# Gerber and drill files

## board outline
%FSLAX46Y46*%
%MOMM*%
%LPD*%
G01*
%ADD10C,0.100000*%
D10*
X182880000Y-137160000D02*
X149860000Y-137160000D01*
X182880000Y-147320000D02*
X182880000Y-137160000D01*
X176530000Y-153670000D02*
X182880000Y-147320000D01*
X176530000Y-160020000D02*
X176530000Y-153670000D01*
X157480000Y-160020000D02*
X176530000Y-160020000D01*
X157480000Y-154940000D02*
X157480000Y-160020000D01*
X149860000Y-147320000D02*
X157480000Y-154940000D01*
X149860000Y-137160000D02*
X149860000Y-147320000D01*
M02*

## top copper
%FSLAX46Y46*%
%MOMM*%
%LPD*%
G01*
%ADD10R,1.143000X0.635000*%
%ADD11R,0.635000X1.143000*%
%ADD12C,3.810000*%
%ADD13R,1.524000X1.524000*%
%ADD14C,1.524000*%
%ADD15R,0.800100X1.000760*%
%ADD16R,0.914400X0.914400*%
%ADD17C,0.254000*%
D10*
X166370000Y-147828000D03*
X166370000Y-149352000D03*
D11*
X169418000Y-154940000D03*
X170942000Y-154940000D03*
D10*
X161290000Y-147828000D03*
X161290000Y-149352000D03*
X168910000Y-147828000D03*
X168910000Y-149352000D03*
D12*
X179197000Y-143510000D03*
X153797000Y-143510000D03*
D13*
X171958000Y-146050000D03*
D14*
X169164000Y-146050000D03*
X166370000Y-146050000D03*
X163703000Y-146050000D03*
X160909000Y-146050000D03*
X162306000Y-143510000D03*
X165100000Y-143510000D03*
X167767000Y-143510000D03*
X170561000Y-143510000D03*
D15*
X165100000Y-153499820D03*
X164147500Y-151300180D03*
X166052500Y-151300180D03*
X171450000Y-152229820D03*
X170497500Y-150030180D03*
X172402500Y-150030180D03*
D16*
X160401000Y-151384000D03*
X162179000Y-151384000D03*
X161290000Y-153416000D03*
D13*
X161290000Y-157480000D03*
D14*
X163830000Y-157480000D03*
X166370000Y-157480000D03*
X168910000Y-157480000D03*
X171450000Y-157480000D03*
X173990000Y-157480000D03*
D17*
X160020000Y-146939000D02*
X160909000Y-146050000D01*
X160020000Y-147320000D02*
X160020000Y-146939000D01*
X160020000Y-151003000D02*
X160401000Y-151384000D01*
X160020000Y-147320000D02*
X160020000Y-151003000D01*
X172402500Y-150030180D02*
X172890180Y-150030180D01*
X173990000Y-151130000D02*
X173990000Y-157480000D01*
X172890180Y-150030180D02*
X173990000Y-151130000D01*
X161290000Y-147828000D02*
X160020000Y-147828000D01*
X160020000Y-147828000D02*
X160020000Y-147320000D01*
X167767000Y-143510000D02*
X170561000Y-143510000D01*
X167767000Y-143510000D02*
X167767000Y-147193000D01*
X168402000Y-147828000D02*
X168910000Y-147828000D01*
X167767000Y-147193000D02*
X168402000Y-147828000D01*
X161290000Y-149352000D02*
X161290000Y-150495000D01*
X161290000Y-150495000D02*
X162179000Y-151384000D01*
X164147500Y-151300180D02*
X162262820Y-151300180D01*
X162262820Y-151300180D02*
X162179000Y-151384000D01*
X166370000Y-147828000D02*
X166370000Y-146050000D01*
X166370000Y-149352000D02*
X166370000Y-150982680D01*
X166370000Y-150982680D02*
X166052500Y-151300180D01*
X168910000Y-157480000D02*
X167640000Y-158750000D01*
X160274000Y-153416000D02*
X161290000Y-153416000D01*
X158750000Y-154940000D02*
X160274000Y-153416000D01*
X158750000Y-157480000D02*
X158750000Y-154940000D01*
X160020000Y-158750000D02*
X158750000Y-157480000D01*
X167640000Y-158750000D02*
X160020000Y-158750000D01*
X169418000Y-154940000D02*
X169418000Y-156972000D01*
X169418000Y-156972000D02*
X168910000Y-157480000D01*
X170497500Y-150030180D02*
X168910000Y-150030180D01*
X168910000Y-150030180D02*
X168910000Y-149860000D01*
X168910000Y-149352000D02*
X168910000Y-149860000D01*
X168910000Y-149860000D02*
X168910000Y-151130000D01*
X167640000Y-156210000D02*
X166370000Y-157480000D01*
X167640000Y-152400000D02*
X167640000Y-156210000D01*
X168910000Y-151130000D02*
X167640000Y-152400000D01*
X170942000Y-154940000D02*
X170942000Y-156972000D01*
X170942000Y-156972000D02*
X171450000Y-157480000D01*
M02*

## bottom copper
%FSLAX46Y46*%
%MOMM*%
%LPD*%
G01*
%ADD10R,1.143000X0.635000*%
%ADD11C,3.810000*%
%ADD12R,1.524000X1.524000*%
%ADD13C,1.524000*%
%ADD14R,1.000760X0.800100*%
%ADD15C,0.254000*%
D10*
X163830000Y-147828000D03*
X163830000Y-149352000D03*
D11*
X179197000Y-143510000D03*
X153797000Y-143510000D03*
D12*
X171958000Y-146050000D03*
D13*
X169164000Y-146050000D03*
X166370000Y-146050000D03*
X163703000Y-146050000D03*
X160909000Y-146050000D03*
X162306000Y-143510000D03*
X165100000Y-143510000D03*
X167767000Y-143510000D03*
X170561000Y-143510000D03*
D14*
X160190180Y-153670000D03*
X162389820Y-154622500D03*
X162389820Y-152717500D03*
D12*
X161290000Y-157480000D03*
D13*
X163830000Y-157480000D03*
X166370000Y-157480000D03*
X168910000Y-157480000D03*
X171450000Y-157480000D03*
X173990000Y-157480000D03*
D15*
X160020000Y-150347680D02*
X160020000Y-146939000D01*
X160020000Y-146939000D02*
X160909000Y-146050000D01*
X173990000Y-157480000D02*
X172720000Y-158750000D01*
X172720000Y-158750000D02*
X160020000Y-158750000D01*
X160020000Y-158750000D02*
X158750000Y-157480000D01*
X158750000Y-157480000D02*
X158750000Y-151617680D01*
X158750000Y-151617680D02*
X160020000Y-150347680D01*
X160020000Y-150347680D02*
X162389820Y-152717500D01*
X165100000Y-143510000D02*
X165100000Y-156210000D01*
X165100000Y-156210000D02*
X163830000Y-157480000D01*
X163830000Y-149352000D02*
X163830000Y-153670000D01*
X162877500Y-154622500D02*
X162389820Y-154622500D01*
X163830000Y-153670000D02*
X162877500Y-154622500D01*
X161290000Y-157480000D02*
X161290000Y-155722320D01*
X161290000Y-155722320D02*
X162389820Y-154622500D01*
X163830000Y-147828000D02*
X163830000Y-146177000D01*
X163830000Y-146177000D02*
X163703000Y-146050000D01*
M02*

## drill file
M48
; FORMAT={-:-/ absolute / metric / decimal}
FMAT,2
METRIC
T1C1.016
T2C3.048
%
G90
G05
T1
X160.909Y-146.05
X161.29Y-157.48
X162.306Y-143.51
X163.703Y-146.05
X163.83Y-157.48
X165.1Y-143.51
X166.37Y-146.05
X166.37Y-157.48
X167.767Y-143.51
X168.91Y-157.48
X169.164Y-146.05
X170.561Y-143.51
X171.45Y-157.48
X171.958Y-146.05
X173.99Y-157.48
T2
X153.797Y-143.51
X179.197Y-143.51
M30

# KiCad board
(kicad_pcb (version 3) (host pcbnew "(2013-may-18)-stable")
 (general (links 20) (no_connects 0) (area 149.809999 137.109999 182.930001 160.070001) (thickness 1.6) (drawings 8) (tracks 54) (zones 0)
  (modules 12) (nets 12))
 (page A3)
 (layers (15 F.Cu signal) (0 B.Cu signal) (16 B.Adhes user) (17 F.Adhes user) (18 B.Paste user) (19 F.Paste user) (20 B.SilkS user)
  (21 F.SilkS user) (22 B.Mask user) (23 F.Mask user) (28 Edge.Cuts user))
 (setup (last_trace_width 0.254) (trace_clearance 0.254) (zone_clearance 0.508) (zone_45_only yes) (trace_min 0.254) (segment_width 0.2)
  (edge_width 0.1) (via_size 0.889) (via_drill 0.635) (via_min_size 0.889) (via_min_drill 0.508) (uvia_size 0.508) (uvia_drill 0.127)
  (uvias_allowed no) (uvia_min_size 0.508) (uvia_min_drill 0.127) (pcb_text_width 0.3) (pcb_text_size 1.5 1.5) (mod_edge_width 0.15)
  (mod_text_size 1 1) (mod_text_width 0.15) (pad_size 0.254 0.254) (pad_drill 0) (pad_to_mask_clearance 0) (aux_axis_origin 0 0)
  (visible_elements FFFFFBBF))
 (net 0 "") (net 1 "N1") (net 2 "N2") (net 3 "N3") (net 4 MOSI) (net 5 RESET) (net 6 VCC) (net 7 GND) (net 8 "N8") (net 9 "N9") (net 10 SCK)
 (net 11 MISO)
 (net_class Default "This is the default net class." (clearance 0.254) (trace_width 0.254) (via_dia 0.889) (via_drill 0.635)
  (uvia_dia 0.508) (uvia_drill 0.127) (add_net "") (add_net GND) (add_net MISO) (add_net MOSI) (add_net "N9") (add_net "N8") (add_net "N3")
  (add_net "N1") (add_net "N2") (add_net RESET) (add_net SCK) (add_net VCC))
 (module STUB (layer F.Cu) (at 0 0)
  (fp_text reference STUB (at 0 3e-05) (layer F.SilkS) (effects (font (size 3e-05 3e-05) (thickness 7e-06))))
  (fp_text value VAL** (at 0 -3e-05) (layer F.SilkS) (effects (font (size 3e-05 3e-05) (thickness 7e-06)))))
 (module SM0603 (layer F.Cu) (at 166.37 148.59 270)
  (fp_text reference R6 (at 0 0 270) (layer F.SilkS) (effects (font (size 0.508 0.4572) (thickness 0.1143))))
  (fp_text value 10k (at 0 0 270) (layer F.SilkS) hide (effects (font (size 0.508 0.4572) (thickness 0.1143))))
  (pad 1 smd rect (at -0.762 0 270) (size 0.635 1.143) (layers F.Cu F.Paste F.Mask) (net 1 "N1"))
  (pad 2 smd rect (at 0.762 0 270) (size 0.635 1.143) (layers F.Cu F.Paste F.Mask) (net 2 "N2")))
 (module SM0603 (layer B.Cu) (at 163.83 148.59 270)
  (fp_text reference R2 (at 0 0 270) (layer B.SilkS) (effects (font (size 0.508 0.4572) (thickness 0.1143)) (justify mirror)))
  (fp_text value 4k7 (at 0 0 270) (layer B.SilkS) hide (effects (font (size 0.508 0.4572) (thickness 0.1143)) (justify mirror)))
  (pad 1 smd rect (at -0.762 0 270) (size 0.635 1.143) (layers B.Cu B.Paste B.Mask) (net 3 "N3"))
  (pad 2 smd rect (at 0.762 0 270) (size 0.635 1.143) (layers B.Cu B.Paste B.Mask) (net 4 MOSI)))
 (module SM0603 (layer F.Cu) (at 170.18 154.94)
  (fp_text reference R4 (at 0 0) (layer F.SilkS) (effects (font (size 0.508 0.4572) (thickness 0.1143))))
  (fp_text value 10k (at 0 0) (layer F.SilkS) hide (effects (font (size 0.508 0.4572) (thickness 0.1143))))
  (pad 1 smd rect (at -0.762 0) (size 0.635 1.143) (layers F.Cu F.Paste F.Mask) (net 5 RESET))
  (pad 2 smd rect (at 0.762 0) (size 0.635 1.143) (layers F.Cu F.Paste F.Mask) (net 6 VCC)))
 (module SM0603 (layer F.Cu) (at 161.29 148.59 270)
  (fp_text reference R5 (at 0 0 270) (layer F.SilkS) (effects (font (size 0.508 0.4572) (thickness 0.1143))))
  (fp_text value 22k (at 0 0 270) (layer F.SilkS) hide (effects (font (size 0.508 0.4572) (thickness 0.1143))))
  (pad 1 smd rect (at -0.762 0 270) (size 0.635 1.143) (layers F.Cu F.Paste F.Mask) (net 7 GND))
  (pad 2 smd rect (at 0.762 0 270) (size 0.635 1.143) (layers F.Cu F.Paste F.Mask) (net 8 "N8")))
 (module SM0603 (layer F.Cu) (at 168.91 148.59 270)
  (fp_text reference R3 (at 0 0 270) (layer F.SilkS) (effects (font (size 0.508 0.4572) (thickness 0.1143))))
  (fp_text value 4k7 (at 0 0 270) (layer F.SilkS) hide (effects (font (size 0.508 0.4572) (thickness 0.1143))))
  (pad 1 smd rect (at -0.762 0 270) (size 0.635 1.143) (layers F.Cu F.Paste F.Mask) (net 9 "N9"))
  (pad 2 smd rect (at 0.762 0 270) (size 0.635 1.143) (layers F.Cu F.Paste F.Mask) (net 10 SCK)))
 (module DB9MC (layer F.Cu) (at 166.37 144.78)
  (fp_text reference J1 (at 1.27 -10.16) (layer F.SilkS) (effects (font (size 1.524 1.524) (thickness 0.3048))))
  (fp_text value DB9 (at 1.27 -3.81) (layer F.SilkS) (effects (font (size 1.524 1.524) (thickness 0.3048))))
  (pad "" thru_hole circle (at 12.827 -1.27) (size 3.81 3.81) (drill 3.048) (layers *.Cu *.Mask F.SilkS))
  (pad "" thru_hole circle (at -12.573 -1.27) (size 3.81 3.81) (drill 3.048) (layers *.Cu *.Mask F.SilkS))
  (pad 1 thru_hole rect (at 5.588 1.27) (size 1.524 1.524) (drill 1.016) (layers *.Cu *.Mask F.SilkS))
  (pad 2 thru_hole circle (at 2.794 1.27) (size 1.524 1.524) (drill 1.016) (layers *.Cu *.Mask F.SilkS))
  (pad 3 thru_hole circle (at 0 1.27) (size 1.524 1.524) (drill 1.016) (layers *.Cu *.Mask F.SilkS) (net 1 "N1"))
  (pad 4 thru_hole circle (at -2.667 1.27) (size 1.524 1.524) (drill 1.016) (layers *.Cu *.Mask F.SilkS) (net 3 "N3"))
  (pad 5 thru_hole circle (at -5.461 1.27) (size 1.524 1.524) (drill 1.016) (layers *.Cu *.Mask F.SilkS) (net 7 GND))
  (pad 9 thru_hole circle (at -4.064 -1.27) (size 1.524 1.524) (drill 1.016) (layers *.Cu *.Mask F.SilkS))
  (pad 8 thru_hole circle (at -1.27 -1.27) (size 1.524 1.524) (drill 1.016) (layers *.Cu *.Mask F.SilkS) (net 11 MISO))
  (pad 7 thru_hole circle (at 1.397 -1.27) (size 1.524 1.524) (drill 1.016) (layers *.Cu *.Mask F.SilkS) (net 9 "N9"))
  (pad 6 thru_hole circle (at 4.191 -1.27) (size 1.524 1.524) (drill 1.016) (layers *.Cu *.Mask F.SilkS) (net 9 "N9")))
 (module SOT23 (layer F.Cu) (at 165.1 152.4 180)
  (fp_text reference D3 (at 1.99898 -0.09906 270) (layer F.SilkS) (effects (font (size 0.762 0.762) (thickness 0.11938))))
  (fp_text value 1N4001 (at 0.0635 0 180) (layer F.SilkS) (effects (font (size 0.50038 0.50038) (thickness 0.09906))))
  (pad 3 smd rect (at 0 -1.09982 180) (size 0.8001 1.00076) (layers F.Cu F.Paste F.Mask))
  (pad 2 smd rect (at 0.9525 1.09982 180) (size 0.8001 1.00076) (layers F.Cu F.Paste F.Mask) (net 8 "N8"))
  (pad 1 smd rect (at -0.9525 1.09982 180) (size 0.8001 1.00076) (layers F.Cu F.Paste F.Mask) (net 2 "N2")))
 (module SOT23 (layer B.Cu) (at 161.29 153.67 270)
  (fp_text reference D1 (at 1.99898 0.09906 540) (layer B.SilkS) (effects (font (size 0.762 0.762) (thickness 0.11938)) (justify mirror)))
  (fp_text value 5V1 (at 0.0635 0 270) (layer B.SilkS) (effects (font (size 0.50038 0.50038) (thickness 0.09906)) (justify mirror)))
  (pad 3 smd rect (at 0 1.09982 270) (size 0.8001 1.00076) (layers B.Cu B.Paste B.Mask))
  (pad 2 smd rect (at 0.9525 -1.09982 270) (size 0.8001 1.00076) (layers B.Cu B.Paste B.Mask) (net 4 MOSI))
  (pad 1 smd rect (at -0.9525 -1.09982 270) (size 0.8001 1.00076) (layers B.Cu B.Paste B.Mask) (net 7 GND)))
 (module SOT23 (layer F.Cu) (at 171.45 151.13 180)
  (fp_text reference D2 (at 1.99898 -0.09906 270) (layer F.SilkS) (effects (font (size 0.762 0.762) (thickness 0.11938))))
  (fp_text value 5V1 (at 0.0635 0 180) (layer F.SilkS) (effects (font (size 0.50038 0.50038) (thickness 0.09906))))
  (pad 3 smd rect (at 0 -1.09982 180) (size 0.8001 1.00076) (layers F.Cu F.Paste F.Mask))
  (pad 2 smd rect (at 0.9525 1.09982 180) (size 0.8001 1.00076) (layers F.Cu F.Paste F.Mask) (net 10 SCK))
  (pad 1 smd rect (at -0.9525 1.09982 180) (size 0.8001 1.00076) (layers F.Cu F.Paste F.Mask) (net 7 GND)))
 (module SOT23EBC (layer F.Cu) (at 161.29 152.4)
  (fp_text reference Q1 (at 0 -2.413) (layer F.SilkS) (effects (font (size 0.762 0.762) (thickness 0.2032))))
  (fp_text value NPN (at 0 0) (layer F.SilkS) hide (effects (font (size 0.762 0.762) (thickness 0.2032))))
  (pad 1 smd rect (at -0.889 -1.016) (size 0.9144 0.9144) (layers F.Cu F.Paste F.Mask) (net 7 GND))
  (pad 2 smd rect (at 0.889 -1.016) (size 0.9144 0.9144) (layers F.Cu F.Paste F.Mask) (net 8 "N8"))
  (pad 3 smd rect (at 0 1.016) (size 0.9144 0.9144) (layers F.Cu F.Paste F.Mask) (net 5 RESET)))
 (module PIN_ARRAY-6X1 (layer F.Cu) (at 167.64 157.48)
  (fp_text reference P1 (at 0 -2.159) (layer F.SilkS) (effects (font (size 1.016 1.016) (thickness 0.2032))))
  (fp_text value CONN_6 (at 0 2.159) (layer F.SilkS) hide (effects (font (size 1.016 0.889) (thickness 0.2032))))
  (pad 1 thru_hole rect (at -6.35 0) (size 1.524 1.524) (drill 1.016) (layers *.Cu *.Mask F.SilkS) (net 4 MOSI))
  (pad 2 thru_hole circle (at -3.81 0) (size 1.524 1.524) (drill 1.016) (layers *.Cu *.Mask F.SilkS) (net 11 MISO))
  (pad 3 thru_hole circle (at -1.27 0) (size 1.524 1.524) (drill 1.016) (layers *.Cu *.Mask F.SilkS) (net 10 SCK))
  (pad 4 thru_hole circle (at 1.27 0) (size 1.524 1.524) (drill 1.016) (layers *.Cu *.Mask F.SilkS) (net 5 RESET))
  (pad 5 thru_hole circle (at 3.81 0) (size 1.524 1.524) (drill 1.016) (layers *.Cu *.Mask F.SilkS) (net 6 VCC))
  (pad 6 thru_hole circle (at 6.35 0) (size 1.524 1.524) (drill 1.016) (layers *.Cu *.Mask F.SilkS) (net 7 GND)))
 (gr_line (start 182.88 137.16) (end 149.86 137.16) (angle 90) (layer Edge.Cuts) (width 0.1))
 (gr_line (start 182.88 147.32) (end 182.88 137.16) (angle 90) (layer Edge.Cuts) (width 0.1))
 (gr_line (start 176.53 153.67) (end 182.88 147.32) (angle 90) (layer Edge.Cuts) (width 0.1))
 (gr_line (start 176.53 160.02) (end 176.53 153.67) (angle 90) (layer Edge.Cuts) (width 0.1))
 (gr_line (start 157.48 160.02) (end 176.53 160.02) (angle 90) (layer Edge.Cuts) (width 0.1))
 (gr_line (start 157.48 154.94) (end 157.48 160.02) (angle 90) (layer Edge.Cuts) (width 0.1))
 (gr_line (start 149.86 147.32) (end 157.48 154.94) (angle 90) (layer Edge.Cuts) (width 0.1))
 (gr_line (start 149.86 137.16) (end 149.86 147.32) (angle 90) (layer Edge.Cuts) (width 0.1))
 (segment (start 160.02 146.939) (end 160.909 146.05) (width 0.254) (layer F.Cu) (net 7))
 (segment (start 160.02 147.32) (end 160.02 146.939) (width 0.254) (layer F.Cu) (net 7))
 (segment (start 160.02 151.003) (end 160.401 151.384) (width 0.254) (layer F.Cu) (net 7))
 (segment (start 160.02 147.32) (end 160.02 151.003) (width 0.254) (layer F.Cu) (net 7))
 (segment (start 160.02 150.34768) (end 160.02 146.939) (width 0.254) (layer B.Cu) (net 7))
 (segment (start 160.02 146.939) (end 160.909 146.05) (width 0.254) (layer B.Cu) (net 7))
 (segment (start 172.4025 150.03018) (end 172.89018 150.03018) (width 0.254) (layer F.Cu) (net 7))
 (segment (start 173.99 151.13) (end 173.99 157.48) (width 0.254) (layer F.Cu) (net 7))
 (segment (start 172.89018 150.03018) (end 173.99 151.13) (width 0.254) (layer F.Cu) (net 7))
 (segment (start 173.99 157.48) (end 172.72 158.75) (width 0.254) (layer B.Cu) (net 7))
 (segment (start 172.72 158.75) (end 160.02 158.75) (width 0.254) (layer B.Cu) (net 7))
 (segment (start 160.02 158.75) (end 158.75 157.48) (width 0.254) (layer B.Cu) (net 7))
 (segment (start 158.75 157.48) (end 158.75 151.61768) (width 0.254) (layer B.Cu) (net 7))
 (segment (start 158.75 151.61768) (end 160.02 150.34768) (width 0.254) (layer B.Cu) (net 7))
 (segment (start 161.29 147.828) (end 160.02 147.828) (width 0.254) (layer F.Cu) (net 7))
 (segment (start 160.02 147.828) (end 160.02 147.32) (width 0.254) (layer F.Cu) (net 7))
 (segment (start 160.02 150.34768) (end 162.38982 152.7175) (width 0.254) (layer B.Cu) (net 7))
 (segment (start 165.1 143.51) (end 165.1 156.21) (width 0.254) (layer B.Cu) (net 11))
 (segment (start 165.1 156.21) (end 163.83 157.48) (width 0.254) (layer B.Cu) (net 11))
 (segment (start 163.83 149.352) (end 163.83 153.67) (width 0.254) (layer B.Cu) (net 4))
 (segment (start 162.8775 154.6225) (end 162.38982 154.6225) (width 0.254) (layer B.Cu) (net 4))
 (segment (start 163.83 153.67) (end 162.8775 154.6225) (width 0.254) (layer B.Cu) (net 4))
 (segment (start 161.29 157.48) (end 161.29 155.72232) (width 0.254) (layer B.Cu) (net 4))
 (segment (start 161.29 155.72232) (end 162.38982 154.6225) (width 0.254) (layer B.Cu) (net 4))
 (segment (start 167.767 143.51) (end 170.561 143.51) (width 0.254) (layer F.Cu) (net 9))
 (segment (start 167.767 143.51) (end 167.767 147.193) (width 0.254) (layer F.Cu) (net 9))
 (segment (start 168.402 147.828) (end 168.91 147.828) (width 0.254) (layer F.Cu) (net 9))
 (segment (start 167.767 147.193) (end 168.402 147.828) (width 0.254) (layer F.Cu) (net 9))
 (segment (start 161.29 149.352) (end 161.29 150.495) (width 0.254) (layer F.Cu) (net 8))
 (segment (start 161.29 150.495) (end 162.179 151.384) (width 0.254) (layer F.Cu) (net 8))
 (segment (start 164.1475 151.30018) (end 162.26282 151.30018) (width 0.254) (layer F.Cu) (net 8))
 (segment (start 162.26282 151.30018) (end 162.179 151.384) (width 0.254) (layer F.Cu) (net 8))
 (segment (start 163.83 147.828) (end 163.83 146.177) (width 0.254) (layer B.Cu) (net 3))
 (segment (start 163.83 146.177) (end 163.703 146.05) (width 0.254) (layer B.Cu) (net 3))
 (segment (start 166.37 147.828) (end 166.37 146.05) (width 0.254) (layer F.Cu) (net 1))
 (segment (start 166.37 149.352) (end 166.37 150.98268) (width 0.254) (layer F.Cu) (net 2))
 (segment (start 166.37 150.98268) (end 166.0525 151.30018) (width 0.254) (layer F.Cu) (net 2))
 (segment (start 168.91 157.48) (end 167.64 158.75) (width 0.254) (layer F.Cu) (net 5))
 (segment (start 160.274 153.416) (end 161.29 153.416) (width 0.254) (layer F.Cu) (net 5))
 (segment (start 158.75 154.94) (end 160.274 153.416) (width 0.254) (layer F.Cu) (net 5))
 (segment (start 158.75 157.48) (end 158.75 154.94) (width 0.254) (layer F.Cu) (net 5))
 (segment (start 160.02 158.75) (end 158.75 157.48) (width 0.254) (layer F.Cu) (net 5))
 (segment (start 167.64 158.75) (end 160.02 158.75) (width 0.254) (layer F.Cu) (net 5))
 (segment (start 169.418 154.94) (end 169.418 156.972) (width 0.254) (layer F.Cu) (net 5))
 (segment (start 169.418 156.972) (end 168.91 157.48) (width 0.254) (layer F.Cu) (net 5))
 (segment (start 170.4975 150.03018) (end 168.91 150.03018) (width 0.254) (layer F.Cu) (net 10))
 (segment (start 168.91 150.03018) (end 168.91 149.86) (width 0.254) (layer F.Cu) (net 10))
 (segment (start 168.91 149.352) (end 168.91 149.86) (width 0.254) (layer F.Cu) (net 10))
 (segment (start 168.91 149.86) (end 168.91 151.13) (width 0.254) (layer F.Cu) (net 10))
 (segment (start 167.64 156.21) (end 166.37 157.48) (width 0.254) (layer F.Cu) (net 10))
 (segment (start 167.64 152.4) (end 167.64 156.21) (width 0.254) (layer F.Cu) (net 10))
 (segment (start 168.91 151.13) (end 167.64 152.4) (width 0.254) (layer F.Cu) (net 10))
 (segment (start 170.942 154.94) (end 170.942 156.972) (width 0.254) (layer F.Cu) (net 6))
 (segment (start 170.942 156.972) (end 171.45 157.48) (width 0.254) (layer F.Cu) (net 6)))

